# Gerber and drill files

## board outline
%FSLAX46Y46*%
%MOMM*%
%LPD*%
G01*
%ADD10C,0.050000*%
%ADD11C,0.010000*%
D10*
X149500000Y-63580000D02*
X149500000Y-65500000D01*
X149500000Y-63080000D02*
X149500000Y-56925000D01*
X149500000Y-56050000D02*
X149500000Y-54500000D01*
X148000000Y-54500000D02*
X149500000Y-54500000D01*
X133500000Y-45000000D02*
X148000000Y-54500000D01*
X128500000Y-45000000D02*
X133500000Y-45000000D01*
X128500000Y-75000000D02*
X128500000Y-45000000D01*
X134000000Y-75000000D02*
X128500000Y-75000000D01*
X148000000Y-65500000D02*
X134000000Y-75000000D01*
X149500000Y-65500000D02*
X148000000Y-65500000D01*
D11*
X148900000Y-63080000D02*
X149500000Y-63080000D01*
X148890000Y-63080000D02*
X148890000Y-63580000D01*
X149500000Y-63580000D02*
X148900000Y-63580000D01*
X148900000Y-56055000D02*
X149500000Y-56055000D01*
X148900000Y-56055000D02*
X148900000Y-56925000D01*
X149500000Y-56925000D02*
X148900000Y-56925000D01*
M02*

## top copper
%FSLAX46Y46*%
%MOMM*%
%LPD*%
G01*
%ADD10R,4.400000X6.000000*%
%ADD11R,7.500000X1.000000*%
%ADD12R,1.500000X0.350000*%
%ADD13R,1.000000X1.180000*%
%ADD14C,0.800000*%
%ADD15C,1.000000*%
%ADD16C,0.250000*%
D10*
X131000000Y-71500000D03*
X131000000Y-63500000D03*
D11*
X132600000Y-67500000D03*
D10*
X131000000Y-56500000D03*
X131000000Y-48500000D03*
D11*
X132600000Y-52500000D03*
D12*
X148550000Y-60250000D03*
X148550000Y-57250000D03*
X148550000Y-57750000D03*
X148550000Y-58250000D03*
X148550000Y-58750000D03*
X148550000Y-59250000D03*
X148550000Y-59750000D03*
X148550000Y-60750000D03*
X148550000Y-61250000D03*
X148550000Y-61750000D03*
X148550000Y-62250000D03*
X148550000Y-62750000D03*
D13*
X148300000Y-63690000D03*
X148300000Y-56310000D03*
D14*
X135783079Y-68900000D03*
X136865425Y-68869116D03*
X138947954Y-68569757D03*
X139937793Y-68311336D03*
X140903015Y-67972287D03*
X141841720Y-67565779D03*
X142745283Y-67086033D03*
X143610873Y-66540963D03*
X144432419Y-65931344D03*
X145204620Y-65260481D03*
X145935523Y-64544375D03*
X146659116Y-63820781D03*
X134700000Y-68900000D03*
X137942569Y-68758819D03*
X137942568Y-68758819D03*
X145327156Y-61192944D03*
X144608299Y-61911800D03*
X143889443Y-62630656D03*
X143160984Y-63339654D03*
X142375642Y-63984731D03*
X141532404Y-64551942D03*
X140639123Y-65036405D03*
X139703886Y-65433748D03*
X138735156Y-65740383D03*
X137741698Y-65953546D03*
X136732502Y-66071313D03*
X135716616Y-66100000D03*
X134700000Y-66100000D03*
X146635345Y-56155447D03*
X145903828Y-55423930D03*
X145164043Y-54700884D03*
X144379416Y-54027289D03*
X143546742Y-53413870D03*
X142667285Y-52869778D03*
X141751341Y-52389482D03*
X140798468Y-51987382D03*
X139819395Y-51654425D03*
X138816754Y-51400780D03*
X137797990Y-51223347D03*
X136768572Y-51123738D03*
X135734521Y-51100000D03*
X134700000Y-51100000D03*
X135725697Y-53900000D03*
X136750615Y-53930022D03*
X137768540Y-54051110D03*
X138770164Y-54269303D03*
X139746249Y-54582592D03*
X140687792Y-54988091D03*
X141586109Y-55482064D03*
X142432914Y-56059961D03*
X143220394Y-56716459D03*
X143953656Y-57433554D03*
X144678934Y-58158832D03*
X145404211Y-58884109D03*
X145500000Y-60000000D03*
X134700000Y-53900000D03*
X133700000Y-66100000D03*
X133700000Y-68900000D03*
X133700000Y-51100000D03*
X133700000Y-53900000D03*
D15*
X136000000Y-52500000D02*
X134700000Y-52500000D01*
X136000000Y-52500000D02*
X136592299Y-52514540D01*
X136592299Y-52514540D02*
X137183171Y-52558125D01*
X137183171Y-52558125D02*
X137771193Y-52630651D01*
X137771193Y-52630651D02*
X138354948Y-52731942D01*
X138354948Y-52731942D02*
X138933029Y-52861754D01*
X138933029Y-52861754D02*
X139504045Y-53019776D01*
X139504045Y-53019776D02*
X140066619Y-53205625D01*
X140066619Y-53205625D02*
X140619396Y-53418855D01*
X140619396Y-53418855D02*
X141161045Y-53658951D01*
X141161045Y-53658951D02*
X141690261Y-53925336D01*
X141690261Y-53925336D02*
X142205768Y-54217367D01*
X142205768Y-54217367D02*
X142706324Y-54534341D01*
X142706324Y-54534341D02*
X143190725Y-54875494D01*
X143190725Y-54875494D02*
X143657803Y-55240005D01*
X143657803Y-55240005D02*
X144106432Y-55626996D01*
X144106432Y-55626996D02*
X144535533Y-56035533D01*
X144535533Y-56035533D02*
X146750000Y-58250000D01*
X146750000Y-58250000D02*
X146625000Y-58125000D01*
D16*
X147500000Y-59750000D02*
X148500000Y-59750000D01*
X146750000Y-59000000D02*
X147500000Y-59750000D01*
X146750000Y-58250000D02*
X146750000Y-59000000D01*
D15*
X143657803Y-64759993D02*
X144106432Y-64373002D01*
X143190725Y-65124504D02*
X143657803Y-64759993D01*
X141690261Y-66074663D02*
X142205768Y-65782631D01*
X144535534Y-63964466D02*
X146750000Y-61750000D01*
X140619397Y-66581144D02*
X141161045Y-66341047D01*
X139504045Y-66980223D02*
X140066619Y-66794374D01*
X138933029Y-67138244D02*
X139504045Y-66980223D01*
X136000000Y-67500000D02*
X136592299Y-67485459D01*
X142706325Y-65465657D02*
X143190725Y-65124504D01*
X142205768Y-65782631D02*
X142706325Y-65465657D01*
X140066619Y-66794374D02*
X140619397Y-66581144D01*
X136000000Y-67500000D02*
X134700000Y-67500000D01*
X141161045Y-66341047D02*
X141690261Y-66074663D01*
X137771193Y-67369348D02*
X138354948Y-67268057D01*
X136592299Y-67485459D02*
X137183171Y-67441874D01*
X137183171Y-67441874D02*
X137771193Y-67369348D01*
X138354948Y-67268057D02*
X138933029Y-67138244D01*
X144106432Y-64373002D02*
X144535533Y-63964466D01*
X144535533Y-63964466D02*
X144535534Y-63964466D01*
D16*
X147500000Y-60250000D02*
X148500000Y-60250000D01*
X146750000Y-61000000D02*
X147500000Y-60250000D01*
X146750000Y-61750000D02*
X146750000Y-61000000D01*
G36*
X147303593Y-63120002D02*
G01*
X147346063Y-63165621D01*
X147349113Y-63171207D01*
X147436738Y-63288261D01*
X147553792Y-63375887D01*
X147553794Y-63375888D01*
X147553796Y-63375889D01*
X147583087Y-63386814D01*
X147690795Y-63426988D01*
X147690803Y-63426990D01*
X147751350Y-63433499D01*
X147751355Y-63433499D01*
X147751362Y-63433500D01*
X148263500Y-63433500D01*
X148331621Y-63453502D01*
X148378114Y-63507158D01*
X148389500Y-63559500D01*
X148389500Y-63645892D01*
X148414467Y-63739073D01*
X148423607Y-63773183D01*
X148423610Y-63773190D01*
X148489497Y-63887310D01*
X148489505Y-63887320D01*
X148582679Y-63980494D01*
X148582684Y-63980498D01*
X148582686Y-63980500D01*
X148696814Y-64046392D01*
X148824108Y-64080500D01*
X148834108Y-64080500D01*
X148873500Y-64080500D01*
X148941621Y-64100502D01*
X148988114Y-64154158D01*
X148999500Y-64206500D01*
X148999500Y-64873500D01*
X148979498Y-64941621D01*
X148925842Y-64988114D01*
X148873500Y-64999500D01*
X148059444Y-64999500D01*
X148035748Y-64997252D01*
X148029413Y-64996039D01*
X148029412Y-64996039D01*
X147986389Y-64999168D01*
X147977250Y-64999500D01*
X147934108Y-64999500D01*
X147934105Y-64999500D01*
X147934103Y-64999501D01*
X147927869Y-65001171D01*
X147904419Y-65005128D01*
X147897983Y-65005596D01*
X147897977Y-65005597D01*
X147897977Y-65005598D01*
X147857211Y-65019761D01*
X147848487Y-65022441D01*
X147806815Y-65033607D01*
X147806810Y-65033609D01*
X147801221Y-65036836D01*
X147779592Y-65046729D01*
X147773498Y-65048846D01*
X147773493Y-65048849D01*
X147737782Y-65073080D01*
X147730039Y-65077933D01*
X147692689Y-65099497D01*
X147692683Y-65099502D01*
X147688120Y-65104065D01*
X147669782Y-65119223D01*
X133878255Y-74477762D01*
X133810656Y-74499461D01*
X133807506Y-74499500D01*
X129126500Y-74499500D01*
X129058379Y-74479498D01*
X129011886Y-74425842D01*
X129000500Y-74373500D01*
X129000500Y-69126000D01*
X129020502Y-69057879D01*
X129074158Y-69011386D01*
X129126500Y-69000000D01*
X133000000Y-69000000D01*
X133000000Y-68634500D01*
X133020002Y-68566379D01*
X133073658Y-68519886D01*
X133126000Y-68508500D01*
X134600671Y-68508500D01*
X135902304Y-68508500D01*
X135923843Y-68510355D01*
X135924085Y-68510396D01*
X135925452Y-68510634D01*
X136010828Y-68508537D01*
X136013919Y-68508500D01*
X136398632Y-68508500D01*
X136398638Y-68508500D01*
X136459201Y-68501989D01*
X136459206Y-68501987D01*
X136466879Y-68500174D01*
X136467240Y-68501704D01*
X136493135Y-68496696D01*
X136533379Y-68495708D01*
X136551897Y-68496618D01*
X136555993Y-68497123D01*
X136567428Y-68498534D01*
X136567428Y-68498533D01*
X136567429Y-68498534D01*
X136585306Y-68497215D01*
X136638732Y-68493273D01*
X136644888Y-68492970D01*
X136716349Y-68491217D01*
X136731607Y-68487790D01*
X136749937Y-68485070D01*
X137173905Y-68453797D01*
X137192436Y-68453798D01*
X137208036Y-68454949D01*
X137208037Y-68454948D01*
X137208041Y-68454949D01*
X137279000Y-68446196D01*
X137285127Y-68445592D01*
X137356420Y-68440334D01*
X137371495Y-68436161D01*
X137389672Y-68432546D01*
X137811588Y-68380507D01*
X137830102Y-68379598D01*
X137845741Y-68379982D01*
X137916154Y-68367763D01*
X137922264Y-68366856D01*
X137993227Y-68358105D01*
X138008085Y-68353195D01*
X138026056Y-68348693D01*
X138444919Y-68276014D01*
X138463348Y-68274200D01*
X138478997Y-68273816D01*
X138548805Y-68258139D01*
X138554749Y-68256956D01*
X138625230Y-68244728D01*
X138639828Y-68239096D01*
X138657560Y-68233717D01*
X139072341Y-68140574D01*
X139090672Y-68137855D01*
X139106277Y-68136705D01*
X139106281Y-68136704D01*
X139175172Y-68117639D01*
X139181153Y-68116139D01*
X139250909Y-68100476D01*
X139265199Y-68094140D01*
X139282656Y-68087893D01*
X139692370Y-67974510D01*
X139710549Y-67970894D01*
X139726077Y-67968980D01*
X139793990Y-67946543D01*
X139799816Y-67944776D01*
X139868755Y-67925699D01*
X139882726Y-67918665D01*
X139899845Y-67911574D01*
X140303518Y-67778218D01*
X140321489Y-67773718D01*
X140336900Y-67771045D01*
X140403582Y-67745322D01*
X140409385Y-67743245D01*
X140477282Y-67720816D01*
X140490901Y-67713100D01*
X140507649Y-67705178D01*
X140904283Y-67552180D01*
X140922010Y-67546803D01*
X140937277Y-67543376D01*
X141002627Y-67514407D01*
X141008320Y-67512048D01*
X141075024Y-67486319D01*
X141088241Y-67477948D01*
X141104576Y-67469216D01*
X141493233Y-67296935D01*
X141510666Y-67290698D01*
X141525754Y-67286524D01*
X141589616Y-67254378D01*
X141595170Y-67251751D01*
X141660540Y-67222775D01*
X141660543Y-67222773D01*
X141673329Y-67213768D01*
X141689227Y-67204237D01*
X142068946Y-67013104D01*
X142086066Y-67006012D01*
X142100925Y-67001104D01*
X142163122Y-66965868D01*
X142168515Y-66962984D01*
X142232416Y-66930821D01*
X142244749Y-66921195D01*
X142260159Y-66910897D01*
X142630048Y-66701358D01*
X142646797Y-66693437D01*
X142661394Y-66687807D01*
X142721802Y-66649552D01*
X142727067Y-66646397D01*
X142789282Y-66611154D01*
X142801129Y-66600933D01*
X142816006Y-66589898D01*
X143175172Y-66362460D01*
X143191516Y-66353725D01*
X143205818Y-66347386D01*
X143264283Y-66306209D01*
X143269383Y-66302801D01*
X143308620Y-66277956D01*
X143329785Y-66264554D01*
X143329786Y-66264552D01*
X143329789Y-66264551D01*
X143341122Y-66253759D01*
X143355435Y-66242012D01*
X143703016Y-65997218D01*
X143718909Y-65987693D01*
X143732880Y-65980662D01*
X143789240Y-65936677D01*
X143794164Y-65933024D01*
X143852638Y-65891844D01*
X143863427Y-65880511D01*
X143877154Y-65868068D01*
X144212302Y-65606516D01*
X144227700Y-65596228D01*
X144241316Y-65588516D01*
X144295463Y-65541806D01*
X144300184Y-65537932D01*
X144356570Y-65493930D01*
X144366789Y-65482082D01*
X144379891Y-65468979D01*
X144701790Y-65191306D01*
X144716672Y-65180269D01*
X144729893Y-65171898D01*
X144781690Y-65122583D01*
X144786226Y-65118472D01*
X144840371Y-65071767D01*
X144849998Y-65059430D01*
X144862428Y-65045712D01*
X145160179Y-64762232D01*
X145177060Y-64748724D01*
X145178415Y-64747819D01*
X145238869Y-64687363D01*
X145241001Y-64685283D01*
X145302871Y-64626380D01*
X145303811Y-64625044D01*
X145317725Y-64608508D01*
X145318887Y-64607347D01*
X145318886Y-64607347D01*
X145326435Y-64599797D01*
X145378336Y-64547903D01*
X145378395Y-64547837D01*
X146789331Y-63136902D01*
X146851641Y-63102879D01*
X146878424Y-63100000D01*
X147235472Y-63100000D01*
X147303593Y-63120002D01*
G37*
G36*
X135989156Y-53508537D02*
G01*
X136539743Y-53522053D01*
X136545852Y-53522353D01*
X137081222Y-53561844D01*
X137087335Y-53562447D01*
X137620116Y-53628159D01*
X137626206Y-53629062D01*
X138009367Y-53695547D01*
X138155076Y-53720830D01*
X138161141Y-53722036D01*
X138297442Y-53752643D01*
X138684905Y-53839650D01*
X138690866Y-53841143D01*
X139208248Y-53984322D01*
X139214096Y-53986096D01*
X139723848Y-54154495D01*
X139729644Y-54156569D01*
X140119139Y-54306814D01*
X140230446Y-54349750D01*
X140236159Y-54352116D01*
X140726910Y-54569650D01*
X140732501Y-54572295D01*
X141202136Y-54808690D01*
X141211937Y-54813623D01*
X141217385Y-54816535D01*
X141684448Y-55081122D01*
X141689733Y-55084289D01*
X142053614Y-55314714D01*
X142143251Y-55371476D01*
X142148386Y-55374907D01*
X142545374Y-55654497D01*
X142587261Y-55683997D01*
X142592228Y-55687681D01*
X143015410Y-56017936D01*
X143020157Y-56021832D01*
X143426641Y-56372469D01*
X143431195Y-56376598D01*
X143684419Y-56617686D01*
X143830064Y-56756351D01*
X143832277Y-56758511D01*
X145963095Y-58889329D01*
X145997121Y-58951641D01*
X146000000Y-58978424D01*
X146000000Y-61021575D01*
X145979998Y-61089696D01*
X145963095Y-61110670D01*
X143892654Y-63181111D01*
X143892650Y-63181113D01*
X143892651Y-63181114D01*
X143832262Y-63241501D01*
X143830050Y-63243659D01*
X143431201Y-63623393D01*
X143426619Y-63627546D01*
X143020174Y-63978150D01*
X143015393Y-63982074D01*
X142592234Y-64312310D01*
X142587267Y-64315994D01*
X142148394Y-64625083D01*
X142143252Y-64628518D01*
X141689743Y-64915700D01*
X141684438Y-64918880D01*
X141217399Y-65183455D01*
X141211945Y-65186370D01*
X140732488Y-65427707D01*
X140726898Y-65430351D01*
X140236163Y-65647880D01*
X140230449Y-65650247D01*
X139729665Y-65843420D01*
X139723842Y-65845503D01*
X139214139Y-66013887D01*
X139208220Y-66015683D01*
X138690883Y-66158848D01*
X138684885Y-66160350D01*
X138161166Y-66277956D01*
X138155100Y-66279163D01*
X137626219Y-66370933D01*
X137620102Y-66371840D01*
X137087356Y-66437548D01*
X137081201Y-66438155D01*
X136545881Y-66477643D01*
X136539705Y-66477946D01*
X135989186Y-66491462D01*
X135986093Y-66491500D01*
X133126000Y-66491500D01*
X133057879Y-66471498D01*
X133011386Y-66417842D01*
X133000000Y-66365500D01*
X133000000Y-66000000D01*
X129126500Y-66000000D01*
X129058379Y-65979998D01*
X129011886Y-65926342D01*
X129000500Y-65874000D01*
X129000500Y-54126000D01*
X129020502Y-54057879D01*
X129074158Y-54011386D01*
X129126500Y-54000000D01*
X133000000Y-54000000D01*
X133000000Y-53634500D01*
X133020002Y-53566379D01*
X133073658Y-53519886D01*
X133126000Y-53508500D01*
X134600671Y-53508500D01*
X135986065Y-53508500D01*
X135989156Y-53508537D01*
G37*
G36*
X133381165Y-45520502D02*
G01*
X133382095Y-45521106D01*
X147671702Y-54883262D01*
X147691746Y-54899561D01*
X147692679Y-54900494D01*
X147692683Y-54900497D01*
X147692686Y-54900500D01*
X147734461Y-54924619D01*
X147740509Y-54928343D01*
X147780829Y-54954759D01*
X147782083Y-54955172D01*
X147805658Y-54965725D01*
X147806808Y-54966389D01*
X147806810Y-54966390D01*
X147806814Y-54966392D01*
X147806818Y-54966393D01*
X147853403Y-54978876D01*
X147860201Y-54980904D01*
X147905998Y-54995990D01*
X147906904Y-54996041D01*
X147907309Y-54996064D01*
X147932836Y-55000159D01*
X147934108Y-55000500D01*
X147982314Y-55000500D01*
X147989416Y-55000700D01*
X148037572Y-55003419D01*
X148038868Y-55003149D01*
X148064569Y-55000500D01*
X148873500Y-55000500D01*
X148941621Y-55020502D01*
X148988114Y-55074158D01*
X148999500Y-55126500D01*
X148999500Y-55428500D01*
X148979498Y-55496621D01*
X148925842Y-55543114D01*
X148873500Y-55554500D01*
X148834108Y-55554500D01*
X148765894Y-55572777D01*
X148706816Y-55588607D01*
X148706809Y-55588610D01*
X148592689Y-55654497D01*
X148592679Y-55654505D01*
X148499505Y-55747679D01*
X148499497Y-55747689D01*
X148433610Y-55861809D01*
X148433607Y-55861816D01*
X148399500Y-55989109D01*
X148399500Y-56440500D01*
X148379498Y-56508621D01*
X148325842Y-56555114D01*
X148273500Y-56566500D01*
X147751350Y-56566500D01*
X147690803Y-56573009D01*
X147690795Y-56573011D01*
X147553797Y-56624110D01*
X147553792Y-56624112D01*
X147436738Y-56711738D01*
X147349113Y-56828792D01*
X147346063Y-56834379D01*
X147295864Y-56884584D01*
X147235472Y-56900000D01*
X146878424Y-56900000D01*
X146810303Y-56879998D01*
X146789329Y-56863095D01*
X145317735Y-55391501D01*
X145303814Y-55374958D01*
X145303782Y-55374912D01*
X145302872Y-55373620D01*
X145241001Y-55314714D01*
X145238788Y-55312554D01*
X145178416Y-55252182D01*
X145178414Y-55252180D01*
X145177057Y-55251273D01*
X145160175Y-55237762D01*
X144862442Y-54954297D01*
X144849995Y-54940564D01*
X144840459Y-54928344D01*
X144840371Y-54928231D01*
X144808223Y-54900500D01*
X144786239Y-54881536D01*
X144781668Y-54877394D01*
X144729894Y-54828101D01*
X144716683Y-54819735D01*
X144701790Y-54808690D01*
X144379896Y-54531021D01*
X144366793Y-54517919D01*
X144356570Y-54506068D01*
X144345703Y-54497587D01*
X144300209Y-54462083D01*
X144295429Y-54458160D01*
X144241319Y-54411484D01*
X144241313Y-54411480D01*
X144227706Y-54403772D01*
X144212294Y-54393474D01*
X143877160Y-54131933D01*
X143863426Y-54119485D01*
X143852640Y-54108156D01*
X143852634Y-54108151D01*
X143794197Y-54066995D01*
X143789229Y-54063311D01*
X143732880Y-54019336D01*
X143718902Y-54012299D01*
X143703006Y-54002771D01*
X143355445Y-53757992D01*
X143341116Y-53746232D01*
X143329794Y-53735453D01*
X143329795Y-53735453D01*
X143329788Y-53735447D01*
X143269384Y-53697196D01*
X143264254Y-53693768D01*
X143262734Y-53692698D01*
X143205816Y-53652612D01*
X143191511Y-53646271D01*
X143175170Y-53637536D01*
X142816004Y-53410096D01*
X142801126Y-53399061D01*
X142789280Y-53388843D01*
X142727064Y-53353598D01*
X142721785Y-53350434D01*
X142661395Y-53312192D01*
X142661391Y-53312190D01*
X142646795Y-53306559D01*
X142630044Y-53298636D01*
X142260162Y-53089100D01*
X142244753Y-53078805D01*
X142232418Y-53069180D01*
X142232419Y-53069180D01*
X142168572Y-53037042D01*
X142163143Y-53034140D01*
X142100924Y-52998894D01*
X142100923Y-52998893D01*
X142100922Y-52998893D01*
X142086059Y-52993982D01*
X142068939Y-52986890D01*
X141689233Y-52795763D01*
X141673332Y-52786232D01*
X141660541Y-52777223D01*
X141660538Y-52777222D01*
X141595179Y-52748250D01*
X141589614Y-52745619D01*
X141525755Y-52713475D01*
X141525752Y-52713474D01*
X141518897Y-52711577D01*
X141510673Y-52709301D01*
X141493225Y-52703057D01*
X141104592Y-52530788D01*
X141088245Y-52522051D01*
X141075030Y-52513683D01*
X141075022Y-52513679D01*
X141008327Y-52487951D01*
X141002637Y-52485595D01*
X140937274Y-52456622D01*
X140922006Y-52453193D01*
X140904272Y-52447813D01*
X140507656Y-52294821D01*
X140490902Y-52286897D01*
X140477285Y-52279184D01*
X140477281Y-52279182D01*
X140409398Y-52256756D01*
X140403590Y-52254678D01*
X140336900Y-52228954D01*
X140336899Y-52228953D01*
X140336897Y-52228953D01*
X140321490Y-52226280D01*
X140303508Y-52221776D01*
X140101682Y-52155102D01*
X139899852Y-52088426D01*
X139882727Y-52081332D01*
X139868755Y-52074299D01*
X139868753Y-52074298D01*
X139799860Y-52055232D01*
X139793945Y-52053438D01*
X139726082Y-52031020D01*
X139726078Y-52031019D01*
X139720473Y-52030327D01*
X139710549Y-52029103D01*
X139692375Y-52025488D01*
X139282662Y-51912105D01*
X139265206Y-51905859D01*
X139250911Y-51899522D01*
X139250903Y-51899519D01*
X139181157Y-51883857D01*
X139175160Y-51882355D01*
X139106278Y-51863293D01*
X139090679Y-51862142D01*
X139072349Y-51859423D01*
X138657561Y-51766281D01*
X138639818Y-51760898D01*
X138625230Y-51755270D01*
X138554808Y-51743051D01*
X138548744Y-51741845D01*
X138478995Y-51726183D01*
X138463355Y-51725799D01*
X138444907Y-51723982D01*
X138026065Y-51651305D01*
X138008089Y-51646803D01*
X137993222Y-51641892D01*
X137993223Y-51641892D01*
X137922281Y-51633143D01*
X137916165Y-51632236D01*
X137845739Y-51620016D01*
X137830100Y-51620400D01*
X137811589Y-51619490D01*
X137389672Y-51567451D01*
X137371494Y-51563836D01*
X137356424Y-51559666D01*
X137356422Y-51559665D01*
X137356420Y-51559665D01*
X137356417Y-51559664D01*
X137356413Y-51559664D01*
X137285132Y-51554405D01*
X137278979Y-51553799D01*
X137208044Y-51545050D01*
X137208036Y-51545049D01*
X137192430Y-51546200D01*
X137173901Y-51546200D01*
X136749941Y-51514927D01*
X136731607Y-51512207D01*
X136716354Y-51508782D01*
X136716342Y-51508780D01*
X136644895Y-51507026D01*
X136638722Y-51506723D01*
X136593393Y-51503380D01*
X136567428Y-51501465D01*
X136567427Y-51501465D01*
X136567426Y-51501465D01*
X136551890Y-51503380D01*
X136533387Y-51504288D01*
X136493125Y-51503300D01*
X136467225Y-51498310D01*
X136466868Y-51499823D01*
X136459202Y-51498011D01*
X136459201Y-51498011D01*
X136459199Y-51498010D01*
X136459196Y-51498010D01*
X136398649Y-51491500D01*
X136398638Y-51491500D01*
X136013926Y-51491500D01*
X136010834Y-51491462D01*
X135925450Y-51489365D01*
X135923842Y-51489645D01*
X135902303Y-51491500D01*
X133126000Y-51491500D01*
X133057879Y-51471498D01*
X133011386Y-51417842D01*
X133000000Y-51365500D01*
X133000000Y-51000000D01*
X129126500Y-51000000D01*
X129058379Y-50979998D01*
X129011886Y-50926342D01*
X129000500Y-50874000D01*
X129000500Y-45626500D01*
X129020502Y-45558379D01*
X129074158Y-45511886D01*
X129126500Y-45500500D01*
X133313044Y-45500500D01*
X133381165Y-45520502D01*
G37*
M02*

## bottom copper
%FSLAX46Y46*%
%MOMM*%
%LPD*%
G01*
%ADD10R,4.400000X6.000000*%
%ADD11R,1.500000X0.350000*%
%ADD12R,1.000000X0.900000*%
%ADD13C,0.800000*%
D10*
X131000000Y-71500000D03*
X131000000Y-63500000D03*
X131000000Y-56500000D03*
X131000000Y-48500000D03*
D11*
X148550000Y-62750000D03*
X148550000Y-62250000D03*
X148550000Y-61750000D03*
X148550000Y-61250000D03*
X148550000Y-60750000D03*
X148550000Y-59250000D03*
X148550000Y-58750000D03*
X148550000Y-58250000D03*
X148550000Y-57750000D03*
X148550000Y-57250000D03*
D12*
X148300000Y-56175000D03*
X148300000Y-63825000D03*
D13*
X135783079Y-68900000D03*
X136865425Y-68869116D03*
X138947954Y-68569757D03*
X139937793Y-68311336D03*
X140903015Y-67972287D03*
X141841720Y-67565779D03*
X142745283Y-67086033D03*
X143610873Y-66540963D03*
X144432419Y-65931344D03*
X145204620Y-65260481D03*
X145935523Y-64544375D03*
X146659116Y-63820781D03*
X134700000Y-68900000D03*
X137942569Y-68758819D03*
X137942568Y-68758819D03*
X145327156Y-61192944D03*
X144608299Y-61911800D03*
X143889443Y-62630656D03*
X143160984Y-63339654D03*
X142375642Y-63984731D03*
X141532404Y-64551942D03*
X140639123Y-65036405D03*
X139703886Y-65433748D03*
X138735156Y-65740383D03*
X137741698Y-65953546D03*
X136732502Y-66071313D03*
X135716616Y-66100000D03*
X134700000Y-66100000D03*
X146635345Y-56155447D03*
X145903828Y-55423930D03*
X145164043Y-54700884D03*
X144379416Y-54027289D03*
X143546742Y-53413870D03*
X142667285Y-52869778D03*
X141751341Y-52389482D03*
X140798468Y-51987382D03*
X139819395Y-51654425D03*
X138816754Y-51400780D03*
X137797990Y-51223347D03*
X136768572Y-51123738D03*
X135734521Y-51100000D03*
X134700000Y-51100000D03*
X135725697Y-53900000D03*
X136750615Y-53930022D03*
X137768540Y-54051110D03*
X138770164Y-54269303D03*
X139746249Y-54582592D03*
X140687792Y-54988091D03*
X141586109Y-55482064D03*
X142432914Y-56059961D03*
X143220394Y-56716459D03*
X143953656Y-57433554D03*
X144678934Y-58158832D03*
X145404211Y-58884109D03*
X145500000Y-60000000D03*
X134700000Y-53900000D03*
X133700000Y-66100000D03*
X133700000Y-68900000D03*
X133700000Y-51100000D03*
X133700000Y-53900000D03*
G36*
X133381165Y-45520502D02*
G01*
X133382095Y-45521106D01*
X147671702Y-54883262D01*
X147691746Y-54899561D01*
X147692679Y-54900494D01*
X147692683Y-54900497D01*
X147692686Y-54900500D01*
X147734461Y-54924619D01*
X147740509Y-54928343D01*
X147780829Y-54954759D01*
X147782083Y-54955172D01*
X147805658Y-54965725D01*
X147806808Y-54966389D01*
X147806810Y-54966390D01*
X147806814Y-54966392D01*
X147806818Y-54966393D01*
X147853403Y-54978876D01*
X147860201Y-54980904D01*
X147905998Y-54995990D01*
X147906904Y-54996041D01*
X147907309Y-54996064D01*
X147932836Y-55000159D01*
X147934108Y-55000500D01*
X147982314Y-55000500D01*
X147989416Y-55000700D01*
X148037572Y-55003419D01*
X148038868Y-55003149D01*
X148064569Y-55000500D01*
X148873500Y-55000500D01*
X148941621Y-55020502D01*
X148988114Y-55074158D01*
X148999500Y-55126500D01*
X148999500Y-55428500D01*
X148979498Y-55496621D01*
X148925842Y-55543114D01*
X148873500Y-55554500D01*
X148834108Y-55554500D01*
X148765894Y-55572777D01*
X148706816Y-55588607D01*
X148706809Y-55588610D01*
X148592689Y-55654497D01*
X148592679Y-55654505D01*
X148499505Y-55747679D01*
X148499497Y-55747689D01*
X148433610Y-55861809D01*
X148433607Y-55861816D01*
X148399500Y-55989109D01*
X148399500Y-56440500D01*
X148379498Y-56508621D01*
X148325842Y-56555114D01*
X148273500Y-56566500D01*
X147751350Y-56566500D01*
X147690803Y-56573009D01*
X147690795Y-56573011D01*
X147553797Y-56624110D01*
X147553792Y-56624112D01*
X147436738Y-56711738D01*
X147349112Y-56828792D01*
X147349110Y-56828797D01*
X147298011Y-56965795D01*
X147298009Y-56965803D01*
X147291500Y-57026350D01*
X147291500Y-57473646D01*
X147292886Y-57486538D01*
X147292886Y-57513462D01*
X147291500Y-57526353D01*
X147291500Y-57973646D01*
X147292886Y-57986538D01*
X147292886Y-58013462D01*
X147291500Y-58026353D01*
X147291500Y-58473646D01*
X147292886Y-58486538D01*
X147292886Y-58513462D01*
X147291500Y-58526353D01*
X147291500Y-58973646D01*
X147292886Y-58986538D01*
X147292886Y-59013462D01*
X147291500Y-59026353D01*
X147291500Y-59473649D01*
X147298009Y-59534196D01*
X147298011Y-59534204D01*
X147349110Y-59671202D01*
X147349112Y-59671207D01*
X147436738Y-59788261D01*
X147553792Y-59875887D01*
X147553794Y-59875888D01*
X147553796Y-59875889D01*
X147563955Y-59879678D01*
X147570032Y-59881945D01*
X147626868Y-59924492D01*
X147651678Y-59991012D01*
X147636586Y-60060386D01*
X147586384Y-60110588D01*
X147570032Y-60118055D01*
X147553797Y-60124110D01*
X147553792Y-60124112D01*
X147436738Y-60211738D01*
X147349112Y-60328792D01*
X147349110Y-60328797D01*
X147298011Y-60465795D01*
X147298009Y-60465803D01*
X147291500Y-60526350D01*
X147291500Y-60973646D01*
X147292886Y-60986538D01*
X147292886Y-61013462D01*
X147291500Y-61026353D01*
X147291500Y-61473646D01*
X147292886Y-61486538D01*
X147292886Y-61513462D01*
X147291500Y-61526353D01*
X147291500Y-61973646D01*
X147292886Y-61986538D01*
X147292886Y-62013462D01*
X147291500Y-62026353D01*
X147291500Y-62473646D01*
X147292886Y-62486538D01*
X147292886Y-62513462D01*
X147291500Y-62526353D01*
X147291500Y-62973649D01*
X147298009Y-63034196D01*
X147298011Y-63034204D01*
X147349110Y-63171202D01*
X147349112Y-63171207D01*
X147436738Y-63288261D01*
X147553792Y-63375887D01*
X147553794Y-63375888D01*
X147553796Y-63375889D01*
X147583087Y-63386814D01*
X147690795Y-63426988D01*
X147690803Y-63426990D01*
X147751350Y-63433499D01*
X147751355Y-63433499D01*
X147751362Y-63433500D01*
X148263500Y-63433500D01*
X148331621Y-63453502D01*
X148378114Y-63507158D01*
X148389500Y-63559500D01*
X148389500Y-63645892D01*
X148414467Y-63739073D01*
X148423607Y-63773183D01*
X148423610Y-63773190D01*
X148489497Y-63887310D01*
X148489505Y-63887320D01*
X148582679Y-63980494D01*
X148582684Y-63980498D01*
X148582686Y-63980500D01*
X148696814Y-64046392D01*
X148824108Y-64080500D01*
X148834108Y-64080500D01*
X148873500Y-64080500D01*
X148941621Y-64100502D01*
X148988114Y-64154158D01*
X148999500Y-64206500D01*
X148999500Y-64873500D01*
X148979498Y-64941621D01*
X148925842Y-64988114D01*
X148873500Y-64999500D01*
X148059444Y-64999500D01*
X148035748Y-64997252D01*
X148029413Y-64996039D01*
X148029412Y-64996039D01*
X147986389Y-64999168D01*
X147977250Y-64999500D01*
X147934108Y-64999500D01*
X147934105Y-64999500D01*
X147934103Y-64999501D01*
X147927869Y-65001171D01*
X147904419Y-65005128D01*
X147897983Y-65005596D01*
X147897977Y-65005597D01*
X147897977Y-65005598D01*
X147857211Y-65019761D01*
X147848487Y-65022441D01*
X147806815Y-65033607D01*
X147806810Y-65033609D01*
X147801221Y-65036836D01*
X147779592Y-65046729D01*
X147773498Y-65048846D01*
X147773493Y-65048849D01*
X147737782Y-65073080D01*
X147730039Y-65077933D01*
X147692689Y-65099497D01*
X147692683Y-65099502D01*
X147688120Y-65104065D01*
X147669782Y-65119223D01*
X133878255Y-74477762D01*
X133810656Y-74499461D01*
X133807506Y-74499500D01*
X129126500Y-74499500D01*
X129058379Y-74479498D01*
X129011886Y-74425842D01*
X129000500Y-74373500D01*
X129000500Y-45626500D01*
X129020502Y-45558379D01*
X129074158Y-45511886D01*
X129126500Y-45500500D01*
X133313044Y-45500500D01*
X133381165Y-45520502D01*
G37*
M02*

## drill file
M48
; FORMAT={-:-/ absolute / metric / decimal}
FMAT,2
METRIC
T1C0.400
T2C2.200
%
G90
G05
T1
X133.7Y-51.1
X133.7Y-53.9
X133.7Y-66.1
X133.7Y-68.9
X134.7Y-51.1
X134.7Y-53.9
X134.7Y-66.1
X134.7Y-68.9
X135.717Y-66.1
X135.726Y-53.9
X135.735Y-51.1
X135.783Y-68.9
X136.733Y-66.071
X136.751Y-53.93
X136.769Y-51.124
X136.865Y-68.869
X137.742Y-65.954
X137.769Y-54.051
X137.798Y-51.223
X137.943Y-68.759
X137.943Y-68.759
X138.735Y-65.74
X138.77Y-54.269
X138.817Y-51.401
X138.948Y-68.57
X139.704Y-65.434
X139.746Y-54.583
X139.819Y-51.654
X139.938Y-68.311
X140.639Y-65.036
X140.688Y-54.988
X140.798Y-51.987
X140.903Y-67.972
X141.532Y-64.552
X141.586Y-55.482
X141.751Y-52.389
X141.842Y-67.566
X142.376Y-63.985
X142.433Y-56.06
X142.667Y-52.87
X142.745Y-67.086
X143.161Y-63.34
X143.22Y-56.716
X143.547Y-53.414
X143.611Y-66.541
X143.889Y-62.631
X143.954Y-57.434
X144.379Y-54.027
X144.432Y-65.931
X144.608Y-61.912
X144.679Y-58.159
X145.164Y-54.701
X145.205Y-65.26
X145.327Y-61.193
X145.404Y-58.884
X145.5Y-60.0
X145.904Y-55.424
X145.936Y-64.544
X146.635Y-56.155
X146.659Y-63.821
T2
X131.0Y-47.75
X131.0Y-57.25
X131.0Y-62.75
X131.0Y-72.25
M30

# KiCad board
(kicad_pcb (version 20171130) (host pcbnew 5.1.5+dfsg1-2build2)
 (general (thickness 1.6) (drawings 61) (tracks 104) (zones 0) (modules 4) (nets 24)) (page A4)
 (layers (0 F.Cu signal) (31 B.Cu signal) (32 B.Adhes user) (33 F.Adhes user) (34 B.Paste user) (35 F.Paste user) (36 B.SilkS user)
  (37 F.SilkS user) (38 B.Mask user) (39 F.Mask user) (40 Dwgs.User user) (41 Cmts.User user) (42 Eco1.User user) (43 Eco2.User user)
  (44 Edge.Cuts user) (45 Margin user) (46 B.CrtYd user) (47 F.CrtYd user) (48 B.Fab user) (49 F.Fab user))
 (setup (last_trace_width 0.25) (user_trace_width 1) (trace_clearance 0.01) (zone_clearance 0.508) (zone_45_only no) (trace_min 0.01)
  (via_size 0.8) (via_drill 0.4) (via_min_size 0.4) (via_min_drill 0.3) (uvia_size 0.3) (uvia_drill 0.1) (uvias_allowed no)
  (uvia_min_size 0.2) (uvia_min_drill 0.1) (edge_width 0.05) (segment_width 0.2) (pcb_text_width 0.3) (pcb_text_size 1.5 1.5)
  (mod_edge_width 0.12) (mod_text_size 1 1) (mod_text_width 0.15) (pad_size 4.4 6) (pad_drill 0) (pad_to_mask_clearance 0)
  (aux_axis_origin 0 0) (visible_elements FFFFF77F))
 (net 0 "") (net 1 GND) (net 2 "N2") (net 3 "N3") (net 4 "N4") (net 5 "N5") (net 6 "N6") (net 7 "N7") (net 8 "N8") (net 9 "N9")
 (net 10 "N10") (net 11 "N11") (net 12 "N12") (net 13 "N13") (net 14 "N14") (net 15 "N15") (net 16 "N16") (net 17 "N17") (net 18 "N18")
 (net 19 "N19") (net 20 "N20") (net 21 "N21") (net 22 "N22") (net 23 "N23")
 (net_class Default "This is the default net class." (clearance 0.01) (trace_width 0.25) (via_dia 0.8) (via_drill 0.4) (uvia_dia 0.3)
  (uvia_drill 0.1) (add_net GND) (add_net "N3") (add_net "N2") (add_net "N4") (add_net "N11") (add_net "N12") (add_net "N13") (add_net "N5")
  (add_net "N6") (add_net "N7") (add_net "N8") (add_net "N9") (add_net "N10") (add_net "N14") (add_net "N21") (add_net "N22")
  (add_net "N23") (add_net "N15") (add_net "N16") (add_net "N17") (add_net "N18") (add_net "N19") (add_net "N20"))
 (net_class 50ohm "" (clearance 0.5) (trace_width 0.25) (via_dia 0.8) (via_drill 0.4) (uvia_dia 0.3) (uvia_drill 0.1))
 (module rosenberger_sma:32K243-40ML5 (layer F.Cu) (at 131 67.5)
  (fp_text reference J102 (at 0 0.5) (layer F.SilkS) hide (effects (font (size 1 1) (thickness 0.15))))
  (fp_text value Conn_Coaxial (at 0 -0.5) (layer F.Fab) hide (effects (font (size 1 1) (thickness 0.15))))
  (pad 2 thru_hole rect (at 0 4.75) (size 4.4 6) (drill 2.2 (offset 0 -0.75)) (layers *.Cu *.Mask) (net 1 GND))
  (pad 2 thru_hole rect (at 0 -4.75) (size 4.4 6) (drill 2.2 (offset 0 0.75)) (layers *.Cu *.Mask) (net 1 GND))
  (pad 1 smd rect (at 1.6 0) (size 7.5 1) (layers F.Cu F.Paste F.Mask) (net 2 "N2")))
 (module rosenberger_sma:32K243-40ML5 (layer F.Cu) (at 131 52.5)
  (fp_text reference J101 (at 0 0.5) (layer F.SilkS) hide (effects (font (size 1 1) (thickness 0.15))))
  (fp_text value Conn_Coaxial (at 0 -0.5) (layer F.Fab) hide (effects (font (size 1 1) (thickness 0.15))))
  (pad 2 thru_hole rect (at 0 4.75) (size 4.4 6) (drill 2.2 (offset 0 -0.75)) (layers *.Cu *.Mask) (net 1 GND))
  (pad 2 thru_hole rect (at 0 -4.75) (size 4.4 6) (drill 2.2 (offset 0 0.75)) (layers *.Cu *.Mask) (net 1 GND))
  (pad 1 smd rect (at 1.6 0) (size 7.5 1) (layers F.Cu F.Paste F.Mask) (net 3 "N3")))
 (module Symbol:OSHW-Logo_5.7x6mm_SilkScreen (layer F.Cu) (at 140 60)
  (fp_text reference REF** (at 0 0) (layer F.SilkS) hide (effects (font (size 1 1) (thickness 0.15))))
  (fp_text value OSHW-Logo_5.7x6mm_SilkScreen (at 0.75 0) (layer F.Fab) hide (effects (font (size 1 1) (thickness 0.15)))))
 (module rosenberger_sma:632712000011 (layer F.Cu) (at 148.55 60 90)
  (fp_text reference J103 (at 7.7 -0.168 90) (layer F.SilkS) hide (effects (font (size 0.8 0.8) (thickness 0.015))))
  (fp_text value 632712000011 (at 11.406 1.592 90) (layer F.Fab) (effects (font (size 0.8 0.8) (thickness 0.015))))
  (fp_line (start -3.08 0.35) (end -3.08 0.95) (layer Edge.Cuts) (width 0.01))
  (fp_line (start -3.08 0.34) (end -3.58 0.34) (layer Edge.Cuts) (width 0.01))
  (fp_line (start -3.58 0.95) (end -3.58 0.35) (layer Edge.Cuts) (width 0.01))
  (fp_line (start 3.945 0.35) (end 3.945 0.95) (layer Edge.Cuts) (width 0.01))
  (fp_line (start 3.945 0.35) (end 3.075 0.35) (layer Edge.Cuts) (width 0.01))
  (fp_line (start 3.075 0.95) (end 3.075 0.35) (layer Edge.Cuts) (width 0.01))
  (pad A7 smd rect (at -0.25 0 90) (size 0.35 1.5) (layers F.Cu F.Paste F.Mask) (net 2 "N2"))
  (pad A1 smd rect (at 2.75 0 90) (size 0.35 1.5) (layers F.Cu F.Paste F.Mask) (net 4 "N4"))
  (pad A2 smd rect (at 2.25 0 90) (size 0.35 1.5) (layers F.Cu F.Paste F.Mask) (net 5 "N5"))
  (pad A3 smd rect (at 1.75 0 90) (size 0.35 1.5) (layers F.Cu F.Paste F.Mask) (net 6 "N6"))
  (pad A4 smd rect (at 1.25 0 90) (size 0.35 1.5) (layers F.Cu F.Paste F.Mask) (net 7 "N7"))
  (pad A5 smd rect (at 0.75 0 90) (size 0.35 1.5) (layers F.Cu F.Paste F.Mask) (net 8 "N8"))
  (pad A6 smd rect (at 0.25 0 90) (size 0.35 1.5) (layers F.Cu F.Paste F.Mask) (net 3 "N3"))
  (pad A8 smd rect (at -0.75 0 90) (size 0.35 1.5) (layers F.Cu F.Paste F.Mask) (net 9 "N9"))
  (pad A9 smd rect (at -1.25 0 90) (size 0.35 1.5) (layers F.Cu F.Paste F.Mask) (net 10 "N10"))
  (pad A10 smd rect (at -1.75 0 90) (size 0.35 1.5) (layers F.Cu F.Paste F.Mask) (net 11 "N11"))
  (pad A11 smd rect (at -2.25 0 90) (size 0.35 1.5) (layers F.Cu F.Paste F.Mask) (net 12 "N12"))
  (pad A12 smd rect (at -2.75 0 90) (size 0.35 1.5) (layers F.Cu F.Paste F.Mask) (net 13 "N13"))
  (pad B1 smd rect (at -2.75 0 90) (size 0.35 1.5) (layers B.Cu B.Paste B.Mask) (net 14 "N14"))
  (pad B2 smd rect (at -2.25 0 90) (size 0.35 1.5) (layers B.Cu B.Paste B.Mask) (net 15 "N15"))
  (pad B3 smd rect (at -1.75 0 90) (size 0.35 1.5) (layers B.Cu B.Paste B.Mask) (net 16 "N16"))
  (pad B4 smd rect (at -1.25 0 90) (size 0.35 1.5) (layers B.Cu B.Paste B.Mask) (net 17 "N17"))
  (pad B5 smd rect (at -0.75 0 90) (size 0.35 1.5) (layers B.Cu B.Paste B.Mask) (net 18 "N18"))
  (pad B8 smd rect (at 0.75 0 90) (size 0.35 1.5) (layers B.Cu B.Paste B.Mask) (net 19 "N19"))
  (pad B9 smd rect (at 1.25 0 90) (size 0.35 1.5) (layers B.Cu B.Paste B.Mask) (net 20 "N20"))
  (pad B10 smd rect (at 1.75 0 90) (size 0.35 1.5) (layers B.Cu B.Paste B.Mask) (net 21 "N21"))
  (pad B11 smd rect (at 2.25 0 90) (size 0.35 1.5) (layers B.Cu B.Paste B.Mask) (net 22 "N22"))
  (pad B12 smd rect (at 2.75 0 90) (size 0.35 1.5) (layers B.Cu B.Paste B.Mask) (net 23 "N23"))
  (pad S4 smd rect (at 3.825 -0.25 90) (size 0.9 1) (layers B.Cu B.Paste B.Mask) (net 1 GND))
  (pad S3 smd rect (at -3.825 -0.25 90) (size 0.9 1) (layers B.Cu B.Paste B.Mask) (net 1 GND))
  (pad S1 smd rect (at -3.69 -0.25 90) (size 1.18 1) (layers F.Cu F.Paste F.Mask) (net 1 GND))
  (pad S2 smd rect (at 3.69 -0.25 90) (size 1.18 1) (layers F.Cu F.Paste F.Mask) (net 1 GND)))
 (gr_line (start 149.5 63.58) (end 149.5 65.5) (layer Edge.Cuts) (width 0.05))
 (gr_line (start 149.5 63.08) (end 149.5 56.925) (layer Edge.Cuts) (width 0.05))
 (gr_line (start 149.5 56.05) (end 149.5 54.5) (layer Edge.Cuts) (width 0.05))
 (gr_line (start 148 54.5) (end 149.5 54.5) (layer Edge.Cuts) (width 0.05))
 (gr_line (start 133.5 45) (end 148 54.5) (layer Edge.Cuts) (width 0.05))
 (gr_line (start 128.5 45) (end 133.5 45) (layer Edge.Cuts) (width 0.05))
 (gr_line (start 128.5 75) (end 128.5 45) (layer Edge.Cuts) (width 0.05))
 (gr_line (start 134 75) (end 128.5 75) (layer Edge.Cuts) (width 0.05))
 (gr_line (start 148 65.5) (end 134 75) (layer Edge.Cuts) (width 0.05))
 (gr_line (start 149.5 65.5) (end 148 65.5) (layer Edge.Cuts) (width 0.05))
 (segment (start 136 52.5) (end 134.7 52.5) (width 1) (layer F.Cu) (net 3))
 (segment (start 136 52.5) (end 136.592299 52.51454) (width 1) (layer F.Cu) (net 3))
 (segment (start 136.592299 52.51454) (end 137.183171 52.558125) (width 1) (layer F.Cu) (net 3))
 (segment (start 137.183171 52.558125) (end 137.771193 52.630651) (width 1) (layer F.Cu) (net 3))
 (segment (start 137.771193 52.630651) (end 138.354948 52.731942) (width 1) (layer F.Cu) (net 3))
 (segment (start 138.354948 52.731942) (end 138.933029 52.861754) (width 1) (layer F.Cu) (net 3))
 (segment (start 138.933029 52.861754) (end 139.504045 53.019776) (width 1) (layer F.Cu) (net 3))
 (segment (start 139.504045 53.019776) (end 140.066619 53.205625) (width 1) (layer F.Cu) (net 3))
 (segment (start 140.066619 53.205625) (end 140.619396 53.418855) (width 1) (layer F.Cu) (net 3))
 (segment (start 140.619396 53.418855) (end 141.161045 53.658951) (width 1) (layer F.Cu) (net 3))
 (segment (start 141.161045 53.658951) (end 141.690261 53.925336) (width 1) (layer F.Cu) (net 3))
 (segment (start 141.690261 53.925336) (end 142.205768 54.217367) (width 1) (layer F.Cu) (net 3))
 (segment (start 142.205768 54.217367) (end 142.706324 54.534341) (width 1) (layer F.Cu) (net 3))
 (segment (start 142.706324 54.534341) (end 143.190725 54.875494) (width 1) (layer F.Cu) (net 3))
 (segment (start 143.190725 54.875494) (end 143.657803 55.240005) (width 1) (layer F.Cu) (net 3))
 (segment (start 143.657803 55.240005) (end 144.106432 55.626996) (width 1) (layer F.Cu) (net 3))
 (segment (start 144.106432 55.626996) (end 144.535533 56.035533) (width 1) (layer F.Cu) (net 3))
 (segment (start 144.535533 56.035533) (end 146.75 58.25) (width 1) (layer F.Cu) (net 3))
 (segment (start 146.75 58.25) (end 146.625 58.125) (width 1) (layer F.Cu) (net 3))
 (segment (start 147.5 59.75) (end 148.5 59.75) (width 0.25) (layer F.Cu) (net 3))
 (segment (start 146.75 59) (end 147.5 59.75) (width 0.25) (layer F.Cu) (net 3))
 (segment (start 146.75 58.25) (end 146.75 59) (width 0.25) (layer F.Cu) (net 3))
 (via (at 135.783079 68.9) (size 0.8) (drill 0.4) (layers F.Cu B.Cu) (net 1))
 (via (at 136.865425 68.869116) (size 0.8) (drill 0.4) (layers F.Cu B.Cu) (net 1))
 (via (at 138.947954 68.569757) (size 0.8) (drill 0.4) (layers F.Cu B.Cu) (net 1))
 (via (at 139.937793 68.311336) (size 0.8) (drill 0.4) (layers F.Cu B.Cu) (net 1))
 (via (at 140.903015 67.972287) (size 0.8) (drill 0.4) (layers F.Cu B.Cu) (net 1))
 (via (at 141.84172 67.565779) (size 0.8) (drill 0.4) (layers F.Cu B.Cu) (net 1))
 (via (at 142.745283 67.086033) (size 0.8) (drill 0.4) (layers F.Cu B.Cu) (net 1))
 (via (at 143.610873 66.540963) (size 0.8) (drill 0.4) (layers F.Cu B.Cu) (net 1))
 (via (at 144.432419 65.931344) (size 0.8) (drill 0.4) (layers F.Cu B.Cu) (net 1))
 (via (at 145.20462 65.260481) (size 0.8) (drill 0.4) (layers F.Cu B.Cu) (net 1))
 (via (at 145.935523 64.544375) (size 0.8) (drill 0.4) (layers F.Cu B.Cu) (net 1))
 (via (at 146.659116 63.820781) (size 0.8) (drill 0.4) (layers F.Cu B.Cu) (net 1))
 (via (at 134.7 68.9) (size 0.8) (drill 0.4) (layers F.Cu B.Cu) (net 1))
 (via (at 137.942569 68.758819) (size 0.8) (drill 0.4) (layers F.Cu B.Cu) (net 1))
 (via (at 137.942568 68.758819) (size 0.8) (drill 0.4) (layers F.Cu B.Cu) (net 1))
 (via (at 145.327156 61.192944) (size 0.8) (drill 0.4) (layers F.Cu B.Cu) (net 1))
 (via (at 144.608299 61.9118) (size 0.8) (drill 0.4) (layers F.Cu B.Cu) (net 1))
 (via (at 143.889443 62.630656) (size 0.8) (drill 0.4) (layers F.Cu B.Cu) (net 1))
 (via (at 143.160984 63.339654) (size 0.8) (drill 0.4) (layers F.Cu B.Cu) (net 1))
 (via (at 142.375642 63.984731) (size 0.8) (drill 0.4) (layers F.Cu B.Cu) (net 1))
 (via (at 141.532404 64.551942) (size 0.8) (drill 0.4) (layers F.Cu B.Cu) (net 1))
 (via (at 140.639123 65.036405) (size 0.8) (drill 0.4) (layers F.Cu B.Cu) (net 1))
 (via (at 139.703886 65.433748) (size 0.8) (drill 0.4) (layers F.Cu B.Cu) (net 1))
 (via (at 138.735156 65.740383) (size 0.8) (drill 0.4) (layers F.Cu B.Cu) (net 1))
 (via (at 137.741698 65.953546) (size 0.8) (drill 0.4) (layers F.Cu B.Cu) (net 1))
 (via (at 136.732502 66.071313) (size 0.8) (drill 0.4) (layers F.Cu B.Cu) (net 1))
 (via (at 135.716616 66.1) (size 0.8) (drill 0.4) (layers F.Cu B.Cu) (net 1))
 (via (at 134.7 66.1) (size 0.8) (drill 0.4) (layers F.Cu B.Cu) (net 1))
 (via (at 146.635345 56.155447) (size 0.8) (drill 0.4) (layers F.Cu B.Cu) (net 1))
 (via (at 145.903828 55.42393) (size 0.8) (drill 0.4) (layers F.Cu B.Cu) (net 1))
 (via (at 145.164043 54.700884) (size 0.8) (drill 0.4) (layers F.Cu B.Cu) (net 1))
 (via (at 144.379416 54.027289) (size 0.8) (drill 0.4) (layers F.Cu B.Cu) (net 1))
 (via (at 143.546742 53.41387) (size 0.8) (drill 0.4) (layers F.Cu B.Cu) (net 1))
 (via (at 142.667285 52.869778) (size 0.8) (drill 0.4) (layers F.Cu B.Cu) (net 1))
 (via (at 141.751341 52.389482) (size 0.8) (drill 0.4) (layers F.Cu B.Cu) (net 1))
 (via (at 140.798468 51.987382) (size 0.8) (drill 0.4) (layers F.Cu B.Cu) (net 1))
 (via (at 139.819395 51.654425) (size 0.8) (drill 0.4) (layers F.Cu B.Cu) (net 1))
 (via (at 138.816754 51.40078) (size 0.8) (drill 0.4) (layers F.Cu B.Cu) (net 1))
 (via (at 137.79799 51.223347) (size 0.8) (drill 0.4) (layers F.Cu B.Cu) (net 1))
 (via (at 136.768572 51.123738) (size 0.8) (drill 0.4) (layers F.Cu B.Cu) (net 1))
 (via (at 135.734521 51.1) (size 0.8) (drill 0.4) (layers F.Cu B.Cu) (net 1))
 (via (at 134.7 51.1) (size 0.8) (drill 0.4) (layers F.Cu B.Cu) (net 1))
 (via (at 135.725697 53.9) (size 0.8) (drill 0.4) (layers F.Cu B.Cu) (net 1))
 (via (at 136.750615 53.930022) (size 0.8) (drill 0.4) (layers F.Cu B.Cu) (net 1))
 (via (at 137.76854 54.05111) (size 0.8) (drill 0.4) (layers F.Cu B.Cu) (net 1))
 (via (at 138.770164 54.269303) (size 0.8) (drill 0.4) (layers F.Cu B.Cu) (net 1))
 (via (at 139.746249 54.582592) (size 0.8) (drill 0.4) (layers F.Cu B.Cu) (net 1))
 (via (at 140.687792 54.988091) (size 0.8) (drill 0.4) (layers F.Cu B.Cu) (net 1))
 (via (at 141.586109 55.482064) (size 0.8) (drill 0.4) (layers F.Cu B.Cu) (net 1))
 (via (at 142.432914 56.059961) (size 0.8) (drill 0.4) (layers F.Cu B.Cu) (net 1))
 (via (at 143.220394 56.716459) (size 0.8) (drill 0.4) (layers F.Cu B.Cu) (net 1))
 (via (at 143.953656 57.433554) (size 0.8) (drill 0.4) (layers F.Cu B.Cu) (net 1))
 (via (at 144.678934 58.158832) (size 0.8) (drill 0.4) (layers F.Cu B.Cu) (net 1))
 (via (at 145.404211 58.884109) (size 0.8) (drill 0.4) (layers F.Cu B.Cu) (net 1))
 (via (at 145.5 60) (size 0.8) (drill 0.4) (layers F.Cu B.Cu) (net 1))
 (via (at 134.7 53.9) (size 0.8) (drill 0.4) (layers F.Cu B.Cu) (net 1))
 (via (at 133.7 66.1) (size 0.8) (drill 0.4) (layers F.Cu B.Cu) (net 1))
 (via (at 133.7 68.9) (size 0.8) (drill 0.4) (layers F.Cu B.Cu) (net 1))
 (via (at 133.7 51.1) (size 0.8) (drill 0.4) (layers F.Cu B.Cu) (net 1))
 (via (at 133.7 53.9) (size 0.8) (drill 0.4) (layers F.Cu B.Cu) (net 1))
 (segment (start 143.657803 64.759993) (end 144.106432 64.373002) (width 1) (layer F.Cu) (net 2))
 (segment (start 143.190725 65.124504) (end 143.657803 64.759993) (width 1) (layer F.Cu) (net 2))
 (segment (start 141.690261 66.074663) (end 142.205768 65.782631) (width 1) (layer F.Cu) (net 2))
 (segment (start 144.535534 63.964466) (end 146.75 61.75) (width 1) (layer F.Cu) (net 2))
 (segment (start 140.619397 66.581144) (end 141.161045 66.341047) (width 1) (layer F.Cu) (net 2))
 (segment (start 139.504045 66.980223) (end 140.066619 66.794374) (width 1) (layer F.Cu) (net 2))
 (segment (start 138.933029 67.138244) (end 139.504045 66.980223) (width 1) (layer F.Cu) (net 2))
 (segment (start 136 67.5) (end 136.592299 67.485459) (width 1) (layer F.Cu) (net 2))
 (segment (start 142.706325 65.465657) (end 143.190725 65.124504) (width 1) (layer F.Cu) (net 2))
 (segment (start 142.205768 65.782631) (end 142.706325 65.465657) (width 1) (layer F.Cu) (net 2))
 (segment (start 140.066619 66.794374) (end 140.619397 66.581144) (width 1) (layer F.Cu) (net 2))
 (segment (start 136 67.5) (end 134.7 67.5) (width 1) (layer F.Cu) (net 2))
 (segment (start 141.161045 66.341047) (end 141.690261 66.074663) (width 1) (layer F.Cu) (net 2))
 (segment (start 137.771193 67.369348) (end 138.354948 67.268057) (width 1) (layer F.Cu) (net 2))
 (segment (start 136.592299 67.485459) (end 137.183171 67.441874) (width 1) (layer F.Cu) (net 2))
 (segment (start 137.183171 67.441874) (end 137.771193 67.369348) (width 1) (layer F.Cu) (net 2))
 (segment (start 138.354948 67.268057) (end 138.933029 67.138244) (width 1) (layer F.Cu) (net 2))
 (segment (start 144.106432 64.373002) (end 144.535533 63.964466) (width 1) (layer F.Cu) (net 2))
 (segment (start 144.535533 63.964466) (end 144.535534 63.964466) (width 1) (layer F.Cu) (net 2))
 (segment (start 147.5 60.25) (end 148.5 60.25) (width 0.25) (layer F.Cu) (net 2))
 (segment (start 146.75 61) (end 147.5 60.25) (width 0.25) (layer F.Cu) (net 2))
 (segment (start 146.75 61.75) (end 146.75 61) (width 0.25) (layer F.Cu) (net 2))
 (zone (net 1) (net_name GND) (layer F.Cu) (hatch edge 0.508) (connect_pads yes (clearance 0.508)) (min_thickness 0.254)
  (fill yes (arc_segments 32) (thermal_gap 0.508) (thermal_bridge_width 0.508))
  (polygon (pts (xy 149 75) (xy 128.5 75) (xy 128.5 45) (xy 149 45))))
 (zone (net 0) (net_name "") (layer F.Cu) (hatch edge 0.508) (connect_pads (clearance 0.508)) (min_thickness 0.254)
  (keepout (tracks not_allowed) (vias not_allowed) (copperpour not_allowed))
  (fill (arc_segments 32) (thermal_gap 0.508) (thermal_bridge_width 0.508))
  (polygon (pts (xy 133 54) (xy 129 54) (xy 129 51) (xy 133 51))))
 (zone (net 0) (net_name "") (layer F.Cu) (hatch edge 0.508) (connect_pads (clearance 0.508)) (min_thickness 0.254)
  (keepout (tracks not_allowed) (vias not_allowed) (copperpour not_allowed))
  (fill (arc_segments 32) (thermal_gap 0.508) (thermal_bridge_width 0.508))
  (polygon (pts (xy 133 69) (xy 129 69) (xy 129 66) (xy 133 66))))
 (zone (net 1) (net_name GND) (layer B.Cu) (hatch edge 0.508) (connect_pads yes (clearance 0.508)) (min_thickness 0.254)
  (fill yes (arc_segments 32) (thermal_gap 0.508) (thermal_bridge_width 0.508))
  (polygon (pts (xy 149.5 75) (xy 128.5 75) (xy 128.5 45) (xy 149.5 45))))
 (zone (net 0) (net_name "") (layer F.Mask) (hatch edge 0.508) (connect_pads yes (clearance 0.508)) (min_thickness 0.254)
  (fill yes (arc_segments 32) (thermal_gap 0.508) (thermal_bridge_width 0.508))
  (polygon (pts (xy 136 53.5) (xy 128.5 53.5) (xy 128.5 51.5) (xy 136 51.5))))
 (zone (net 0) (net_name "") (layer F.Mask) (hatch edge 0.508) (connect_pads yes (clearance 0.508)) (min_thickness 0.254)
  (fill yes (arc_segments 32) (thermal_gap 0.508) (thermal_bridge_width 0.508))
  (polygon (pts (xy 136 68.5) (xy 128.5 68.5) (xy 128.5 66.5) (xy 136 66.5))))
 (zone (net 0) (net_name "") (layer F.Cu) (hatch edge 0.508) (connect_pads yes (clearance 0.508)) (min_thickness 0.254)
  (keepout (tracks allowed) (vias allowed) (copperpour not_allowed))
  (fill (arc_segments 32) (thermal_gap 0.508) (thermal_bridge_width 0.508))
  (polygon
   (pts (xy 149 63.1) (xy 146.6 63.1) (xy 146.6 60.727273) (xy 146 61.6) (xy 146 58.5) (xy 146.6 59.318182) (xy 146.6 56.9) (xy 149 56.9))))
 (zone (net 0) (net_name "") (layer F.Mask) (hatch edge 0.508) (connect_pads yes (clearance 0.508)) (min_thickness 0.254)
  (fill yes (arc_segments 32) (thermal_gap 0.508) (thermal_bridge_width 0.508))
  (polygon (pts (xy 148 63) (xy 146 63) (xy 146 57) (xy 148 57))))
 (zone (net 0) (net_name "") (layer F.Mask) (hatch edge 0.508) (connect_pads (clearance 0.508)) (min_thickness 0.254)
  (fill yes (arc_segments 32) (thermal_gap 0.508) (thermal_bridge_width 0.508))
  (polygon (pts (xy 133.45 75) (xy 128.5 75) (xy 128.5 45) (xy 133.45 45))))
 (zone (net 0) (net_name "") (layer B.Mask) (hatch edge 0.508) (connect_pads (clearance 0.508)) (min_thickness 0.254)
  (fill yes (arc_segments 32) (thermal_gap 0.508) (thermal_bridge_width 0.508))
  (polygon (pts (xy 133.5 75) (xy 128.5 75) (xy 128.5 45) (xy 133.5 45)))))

